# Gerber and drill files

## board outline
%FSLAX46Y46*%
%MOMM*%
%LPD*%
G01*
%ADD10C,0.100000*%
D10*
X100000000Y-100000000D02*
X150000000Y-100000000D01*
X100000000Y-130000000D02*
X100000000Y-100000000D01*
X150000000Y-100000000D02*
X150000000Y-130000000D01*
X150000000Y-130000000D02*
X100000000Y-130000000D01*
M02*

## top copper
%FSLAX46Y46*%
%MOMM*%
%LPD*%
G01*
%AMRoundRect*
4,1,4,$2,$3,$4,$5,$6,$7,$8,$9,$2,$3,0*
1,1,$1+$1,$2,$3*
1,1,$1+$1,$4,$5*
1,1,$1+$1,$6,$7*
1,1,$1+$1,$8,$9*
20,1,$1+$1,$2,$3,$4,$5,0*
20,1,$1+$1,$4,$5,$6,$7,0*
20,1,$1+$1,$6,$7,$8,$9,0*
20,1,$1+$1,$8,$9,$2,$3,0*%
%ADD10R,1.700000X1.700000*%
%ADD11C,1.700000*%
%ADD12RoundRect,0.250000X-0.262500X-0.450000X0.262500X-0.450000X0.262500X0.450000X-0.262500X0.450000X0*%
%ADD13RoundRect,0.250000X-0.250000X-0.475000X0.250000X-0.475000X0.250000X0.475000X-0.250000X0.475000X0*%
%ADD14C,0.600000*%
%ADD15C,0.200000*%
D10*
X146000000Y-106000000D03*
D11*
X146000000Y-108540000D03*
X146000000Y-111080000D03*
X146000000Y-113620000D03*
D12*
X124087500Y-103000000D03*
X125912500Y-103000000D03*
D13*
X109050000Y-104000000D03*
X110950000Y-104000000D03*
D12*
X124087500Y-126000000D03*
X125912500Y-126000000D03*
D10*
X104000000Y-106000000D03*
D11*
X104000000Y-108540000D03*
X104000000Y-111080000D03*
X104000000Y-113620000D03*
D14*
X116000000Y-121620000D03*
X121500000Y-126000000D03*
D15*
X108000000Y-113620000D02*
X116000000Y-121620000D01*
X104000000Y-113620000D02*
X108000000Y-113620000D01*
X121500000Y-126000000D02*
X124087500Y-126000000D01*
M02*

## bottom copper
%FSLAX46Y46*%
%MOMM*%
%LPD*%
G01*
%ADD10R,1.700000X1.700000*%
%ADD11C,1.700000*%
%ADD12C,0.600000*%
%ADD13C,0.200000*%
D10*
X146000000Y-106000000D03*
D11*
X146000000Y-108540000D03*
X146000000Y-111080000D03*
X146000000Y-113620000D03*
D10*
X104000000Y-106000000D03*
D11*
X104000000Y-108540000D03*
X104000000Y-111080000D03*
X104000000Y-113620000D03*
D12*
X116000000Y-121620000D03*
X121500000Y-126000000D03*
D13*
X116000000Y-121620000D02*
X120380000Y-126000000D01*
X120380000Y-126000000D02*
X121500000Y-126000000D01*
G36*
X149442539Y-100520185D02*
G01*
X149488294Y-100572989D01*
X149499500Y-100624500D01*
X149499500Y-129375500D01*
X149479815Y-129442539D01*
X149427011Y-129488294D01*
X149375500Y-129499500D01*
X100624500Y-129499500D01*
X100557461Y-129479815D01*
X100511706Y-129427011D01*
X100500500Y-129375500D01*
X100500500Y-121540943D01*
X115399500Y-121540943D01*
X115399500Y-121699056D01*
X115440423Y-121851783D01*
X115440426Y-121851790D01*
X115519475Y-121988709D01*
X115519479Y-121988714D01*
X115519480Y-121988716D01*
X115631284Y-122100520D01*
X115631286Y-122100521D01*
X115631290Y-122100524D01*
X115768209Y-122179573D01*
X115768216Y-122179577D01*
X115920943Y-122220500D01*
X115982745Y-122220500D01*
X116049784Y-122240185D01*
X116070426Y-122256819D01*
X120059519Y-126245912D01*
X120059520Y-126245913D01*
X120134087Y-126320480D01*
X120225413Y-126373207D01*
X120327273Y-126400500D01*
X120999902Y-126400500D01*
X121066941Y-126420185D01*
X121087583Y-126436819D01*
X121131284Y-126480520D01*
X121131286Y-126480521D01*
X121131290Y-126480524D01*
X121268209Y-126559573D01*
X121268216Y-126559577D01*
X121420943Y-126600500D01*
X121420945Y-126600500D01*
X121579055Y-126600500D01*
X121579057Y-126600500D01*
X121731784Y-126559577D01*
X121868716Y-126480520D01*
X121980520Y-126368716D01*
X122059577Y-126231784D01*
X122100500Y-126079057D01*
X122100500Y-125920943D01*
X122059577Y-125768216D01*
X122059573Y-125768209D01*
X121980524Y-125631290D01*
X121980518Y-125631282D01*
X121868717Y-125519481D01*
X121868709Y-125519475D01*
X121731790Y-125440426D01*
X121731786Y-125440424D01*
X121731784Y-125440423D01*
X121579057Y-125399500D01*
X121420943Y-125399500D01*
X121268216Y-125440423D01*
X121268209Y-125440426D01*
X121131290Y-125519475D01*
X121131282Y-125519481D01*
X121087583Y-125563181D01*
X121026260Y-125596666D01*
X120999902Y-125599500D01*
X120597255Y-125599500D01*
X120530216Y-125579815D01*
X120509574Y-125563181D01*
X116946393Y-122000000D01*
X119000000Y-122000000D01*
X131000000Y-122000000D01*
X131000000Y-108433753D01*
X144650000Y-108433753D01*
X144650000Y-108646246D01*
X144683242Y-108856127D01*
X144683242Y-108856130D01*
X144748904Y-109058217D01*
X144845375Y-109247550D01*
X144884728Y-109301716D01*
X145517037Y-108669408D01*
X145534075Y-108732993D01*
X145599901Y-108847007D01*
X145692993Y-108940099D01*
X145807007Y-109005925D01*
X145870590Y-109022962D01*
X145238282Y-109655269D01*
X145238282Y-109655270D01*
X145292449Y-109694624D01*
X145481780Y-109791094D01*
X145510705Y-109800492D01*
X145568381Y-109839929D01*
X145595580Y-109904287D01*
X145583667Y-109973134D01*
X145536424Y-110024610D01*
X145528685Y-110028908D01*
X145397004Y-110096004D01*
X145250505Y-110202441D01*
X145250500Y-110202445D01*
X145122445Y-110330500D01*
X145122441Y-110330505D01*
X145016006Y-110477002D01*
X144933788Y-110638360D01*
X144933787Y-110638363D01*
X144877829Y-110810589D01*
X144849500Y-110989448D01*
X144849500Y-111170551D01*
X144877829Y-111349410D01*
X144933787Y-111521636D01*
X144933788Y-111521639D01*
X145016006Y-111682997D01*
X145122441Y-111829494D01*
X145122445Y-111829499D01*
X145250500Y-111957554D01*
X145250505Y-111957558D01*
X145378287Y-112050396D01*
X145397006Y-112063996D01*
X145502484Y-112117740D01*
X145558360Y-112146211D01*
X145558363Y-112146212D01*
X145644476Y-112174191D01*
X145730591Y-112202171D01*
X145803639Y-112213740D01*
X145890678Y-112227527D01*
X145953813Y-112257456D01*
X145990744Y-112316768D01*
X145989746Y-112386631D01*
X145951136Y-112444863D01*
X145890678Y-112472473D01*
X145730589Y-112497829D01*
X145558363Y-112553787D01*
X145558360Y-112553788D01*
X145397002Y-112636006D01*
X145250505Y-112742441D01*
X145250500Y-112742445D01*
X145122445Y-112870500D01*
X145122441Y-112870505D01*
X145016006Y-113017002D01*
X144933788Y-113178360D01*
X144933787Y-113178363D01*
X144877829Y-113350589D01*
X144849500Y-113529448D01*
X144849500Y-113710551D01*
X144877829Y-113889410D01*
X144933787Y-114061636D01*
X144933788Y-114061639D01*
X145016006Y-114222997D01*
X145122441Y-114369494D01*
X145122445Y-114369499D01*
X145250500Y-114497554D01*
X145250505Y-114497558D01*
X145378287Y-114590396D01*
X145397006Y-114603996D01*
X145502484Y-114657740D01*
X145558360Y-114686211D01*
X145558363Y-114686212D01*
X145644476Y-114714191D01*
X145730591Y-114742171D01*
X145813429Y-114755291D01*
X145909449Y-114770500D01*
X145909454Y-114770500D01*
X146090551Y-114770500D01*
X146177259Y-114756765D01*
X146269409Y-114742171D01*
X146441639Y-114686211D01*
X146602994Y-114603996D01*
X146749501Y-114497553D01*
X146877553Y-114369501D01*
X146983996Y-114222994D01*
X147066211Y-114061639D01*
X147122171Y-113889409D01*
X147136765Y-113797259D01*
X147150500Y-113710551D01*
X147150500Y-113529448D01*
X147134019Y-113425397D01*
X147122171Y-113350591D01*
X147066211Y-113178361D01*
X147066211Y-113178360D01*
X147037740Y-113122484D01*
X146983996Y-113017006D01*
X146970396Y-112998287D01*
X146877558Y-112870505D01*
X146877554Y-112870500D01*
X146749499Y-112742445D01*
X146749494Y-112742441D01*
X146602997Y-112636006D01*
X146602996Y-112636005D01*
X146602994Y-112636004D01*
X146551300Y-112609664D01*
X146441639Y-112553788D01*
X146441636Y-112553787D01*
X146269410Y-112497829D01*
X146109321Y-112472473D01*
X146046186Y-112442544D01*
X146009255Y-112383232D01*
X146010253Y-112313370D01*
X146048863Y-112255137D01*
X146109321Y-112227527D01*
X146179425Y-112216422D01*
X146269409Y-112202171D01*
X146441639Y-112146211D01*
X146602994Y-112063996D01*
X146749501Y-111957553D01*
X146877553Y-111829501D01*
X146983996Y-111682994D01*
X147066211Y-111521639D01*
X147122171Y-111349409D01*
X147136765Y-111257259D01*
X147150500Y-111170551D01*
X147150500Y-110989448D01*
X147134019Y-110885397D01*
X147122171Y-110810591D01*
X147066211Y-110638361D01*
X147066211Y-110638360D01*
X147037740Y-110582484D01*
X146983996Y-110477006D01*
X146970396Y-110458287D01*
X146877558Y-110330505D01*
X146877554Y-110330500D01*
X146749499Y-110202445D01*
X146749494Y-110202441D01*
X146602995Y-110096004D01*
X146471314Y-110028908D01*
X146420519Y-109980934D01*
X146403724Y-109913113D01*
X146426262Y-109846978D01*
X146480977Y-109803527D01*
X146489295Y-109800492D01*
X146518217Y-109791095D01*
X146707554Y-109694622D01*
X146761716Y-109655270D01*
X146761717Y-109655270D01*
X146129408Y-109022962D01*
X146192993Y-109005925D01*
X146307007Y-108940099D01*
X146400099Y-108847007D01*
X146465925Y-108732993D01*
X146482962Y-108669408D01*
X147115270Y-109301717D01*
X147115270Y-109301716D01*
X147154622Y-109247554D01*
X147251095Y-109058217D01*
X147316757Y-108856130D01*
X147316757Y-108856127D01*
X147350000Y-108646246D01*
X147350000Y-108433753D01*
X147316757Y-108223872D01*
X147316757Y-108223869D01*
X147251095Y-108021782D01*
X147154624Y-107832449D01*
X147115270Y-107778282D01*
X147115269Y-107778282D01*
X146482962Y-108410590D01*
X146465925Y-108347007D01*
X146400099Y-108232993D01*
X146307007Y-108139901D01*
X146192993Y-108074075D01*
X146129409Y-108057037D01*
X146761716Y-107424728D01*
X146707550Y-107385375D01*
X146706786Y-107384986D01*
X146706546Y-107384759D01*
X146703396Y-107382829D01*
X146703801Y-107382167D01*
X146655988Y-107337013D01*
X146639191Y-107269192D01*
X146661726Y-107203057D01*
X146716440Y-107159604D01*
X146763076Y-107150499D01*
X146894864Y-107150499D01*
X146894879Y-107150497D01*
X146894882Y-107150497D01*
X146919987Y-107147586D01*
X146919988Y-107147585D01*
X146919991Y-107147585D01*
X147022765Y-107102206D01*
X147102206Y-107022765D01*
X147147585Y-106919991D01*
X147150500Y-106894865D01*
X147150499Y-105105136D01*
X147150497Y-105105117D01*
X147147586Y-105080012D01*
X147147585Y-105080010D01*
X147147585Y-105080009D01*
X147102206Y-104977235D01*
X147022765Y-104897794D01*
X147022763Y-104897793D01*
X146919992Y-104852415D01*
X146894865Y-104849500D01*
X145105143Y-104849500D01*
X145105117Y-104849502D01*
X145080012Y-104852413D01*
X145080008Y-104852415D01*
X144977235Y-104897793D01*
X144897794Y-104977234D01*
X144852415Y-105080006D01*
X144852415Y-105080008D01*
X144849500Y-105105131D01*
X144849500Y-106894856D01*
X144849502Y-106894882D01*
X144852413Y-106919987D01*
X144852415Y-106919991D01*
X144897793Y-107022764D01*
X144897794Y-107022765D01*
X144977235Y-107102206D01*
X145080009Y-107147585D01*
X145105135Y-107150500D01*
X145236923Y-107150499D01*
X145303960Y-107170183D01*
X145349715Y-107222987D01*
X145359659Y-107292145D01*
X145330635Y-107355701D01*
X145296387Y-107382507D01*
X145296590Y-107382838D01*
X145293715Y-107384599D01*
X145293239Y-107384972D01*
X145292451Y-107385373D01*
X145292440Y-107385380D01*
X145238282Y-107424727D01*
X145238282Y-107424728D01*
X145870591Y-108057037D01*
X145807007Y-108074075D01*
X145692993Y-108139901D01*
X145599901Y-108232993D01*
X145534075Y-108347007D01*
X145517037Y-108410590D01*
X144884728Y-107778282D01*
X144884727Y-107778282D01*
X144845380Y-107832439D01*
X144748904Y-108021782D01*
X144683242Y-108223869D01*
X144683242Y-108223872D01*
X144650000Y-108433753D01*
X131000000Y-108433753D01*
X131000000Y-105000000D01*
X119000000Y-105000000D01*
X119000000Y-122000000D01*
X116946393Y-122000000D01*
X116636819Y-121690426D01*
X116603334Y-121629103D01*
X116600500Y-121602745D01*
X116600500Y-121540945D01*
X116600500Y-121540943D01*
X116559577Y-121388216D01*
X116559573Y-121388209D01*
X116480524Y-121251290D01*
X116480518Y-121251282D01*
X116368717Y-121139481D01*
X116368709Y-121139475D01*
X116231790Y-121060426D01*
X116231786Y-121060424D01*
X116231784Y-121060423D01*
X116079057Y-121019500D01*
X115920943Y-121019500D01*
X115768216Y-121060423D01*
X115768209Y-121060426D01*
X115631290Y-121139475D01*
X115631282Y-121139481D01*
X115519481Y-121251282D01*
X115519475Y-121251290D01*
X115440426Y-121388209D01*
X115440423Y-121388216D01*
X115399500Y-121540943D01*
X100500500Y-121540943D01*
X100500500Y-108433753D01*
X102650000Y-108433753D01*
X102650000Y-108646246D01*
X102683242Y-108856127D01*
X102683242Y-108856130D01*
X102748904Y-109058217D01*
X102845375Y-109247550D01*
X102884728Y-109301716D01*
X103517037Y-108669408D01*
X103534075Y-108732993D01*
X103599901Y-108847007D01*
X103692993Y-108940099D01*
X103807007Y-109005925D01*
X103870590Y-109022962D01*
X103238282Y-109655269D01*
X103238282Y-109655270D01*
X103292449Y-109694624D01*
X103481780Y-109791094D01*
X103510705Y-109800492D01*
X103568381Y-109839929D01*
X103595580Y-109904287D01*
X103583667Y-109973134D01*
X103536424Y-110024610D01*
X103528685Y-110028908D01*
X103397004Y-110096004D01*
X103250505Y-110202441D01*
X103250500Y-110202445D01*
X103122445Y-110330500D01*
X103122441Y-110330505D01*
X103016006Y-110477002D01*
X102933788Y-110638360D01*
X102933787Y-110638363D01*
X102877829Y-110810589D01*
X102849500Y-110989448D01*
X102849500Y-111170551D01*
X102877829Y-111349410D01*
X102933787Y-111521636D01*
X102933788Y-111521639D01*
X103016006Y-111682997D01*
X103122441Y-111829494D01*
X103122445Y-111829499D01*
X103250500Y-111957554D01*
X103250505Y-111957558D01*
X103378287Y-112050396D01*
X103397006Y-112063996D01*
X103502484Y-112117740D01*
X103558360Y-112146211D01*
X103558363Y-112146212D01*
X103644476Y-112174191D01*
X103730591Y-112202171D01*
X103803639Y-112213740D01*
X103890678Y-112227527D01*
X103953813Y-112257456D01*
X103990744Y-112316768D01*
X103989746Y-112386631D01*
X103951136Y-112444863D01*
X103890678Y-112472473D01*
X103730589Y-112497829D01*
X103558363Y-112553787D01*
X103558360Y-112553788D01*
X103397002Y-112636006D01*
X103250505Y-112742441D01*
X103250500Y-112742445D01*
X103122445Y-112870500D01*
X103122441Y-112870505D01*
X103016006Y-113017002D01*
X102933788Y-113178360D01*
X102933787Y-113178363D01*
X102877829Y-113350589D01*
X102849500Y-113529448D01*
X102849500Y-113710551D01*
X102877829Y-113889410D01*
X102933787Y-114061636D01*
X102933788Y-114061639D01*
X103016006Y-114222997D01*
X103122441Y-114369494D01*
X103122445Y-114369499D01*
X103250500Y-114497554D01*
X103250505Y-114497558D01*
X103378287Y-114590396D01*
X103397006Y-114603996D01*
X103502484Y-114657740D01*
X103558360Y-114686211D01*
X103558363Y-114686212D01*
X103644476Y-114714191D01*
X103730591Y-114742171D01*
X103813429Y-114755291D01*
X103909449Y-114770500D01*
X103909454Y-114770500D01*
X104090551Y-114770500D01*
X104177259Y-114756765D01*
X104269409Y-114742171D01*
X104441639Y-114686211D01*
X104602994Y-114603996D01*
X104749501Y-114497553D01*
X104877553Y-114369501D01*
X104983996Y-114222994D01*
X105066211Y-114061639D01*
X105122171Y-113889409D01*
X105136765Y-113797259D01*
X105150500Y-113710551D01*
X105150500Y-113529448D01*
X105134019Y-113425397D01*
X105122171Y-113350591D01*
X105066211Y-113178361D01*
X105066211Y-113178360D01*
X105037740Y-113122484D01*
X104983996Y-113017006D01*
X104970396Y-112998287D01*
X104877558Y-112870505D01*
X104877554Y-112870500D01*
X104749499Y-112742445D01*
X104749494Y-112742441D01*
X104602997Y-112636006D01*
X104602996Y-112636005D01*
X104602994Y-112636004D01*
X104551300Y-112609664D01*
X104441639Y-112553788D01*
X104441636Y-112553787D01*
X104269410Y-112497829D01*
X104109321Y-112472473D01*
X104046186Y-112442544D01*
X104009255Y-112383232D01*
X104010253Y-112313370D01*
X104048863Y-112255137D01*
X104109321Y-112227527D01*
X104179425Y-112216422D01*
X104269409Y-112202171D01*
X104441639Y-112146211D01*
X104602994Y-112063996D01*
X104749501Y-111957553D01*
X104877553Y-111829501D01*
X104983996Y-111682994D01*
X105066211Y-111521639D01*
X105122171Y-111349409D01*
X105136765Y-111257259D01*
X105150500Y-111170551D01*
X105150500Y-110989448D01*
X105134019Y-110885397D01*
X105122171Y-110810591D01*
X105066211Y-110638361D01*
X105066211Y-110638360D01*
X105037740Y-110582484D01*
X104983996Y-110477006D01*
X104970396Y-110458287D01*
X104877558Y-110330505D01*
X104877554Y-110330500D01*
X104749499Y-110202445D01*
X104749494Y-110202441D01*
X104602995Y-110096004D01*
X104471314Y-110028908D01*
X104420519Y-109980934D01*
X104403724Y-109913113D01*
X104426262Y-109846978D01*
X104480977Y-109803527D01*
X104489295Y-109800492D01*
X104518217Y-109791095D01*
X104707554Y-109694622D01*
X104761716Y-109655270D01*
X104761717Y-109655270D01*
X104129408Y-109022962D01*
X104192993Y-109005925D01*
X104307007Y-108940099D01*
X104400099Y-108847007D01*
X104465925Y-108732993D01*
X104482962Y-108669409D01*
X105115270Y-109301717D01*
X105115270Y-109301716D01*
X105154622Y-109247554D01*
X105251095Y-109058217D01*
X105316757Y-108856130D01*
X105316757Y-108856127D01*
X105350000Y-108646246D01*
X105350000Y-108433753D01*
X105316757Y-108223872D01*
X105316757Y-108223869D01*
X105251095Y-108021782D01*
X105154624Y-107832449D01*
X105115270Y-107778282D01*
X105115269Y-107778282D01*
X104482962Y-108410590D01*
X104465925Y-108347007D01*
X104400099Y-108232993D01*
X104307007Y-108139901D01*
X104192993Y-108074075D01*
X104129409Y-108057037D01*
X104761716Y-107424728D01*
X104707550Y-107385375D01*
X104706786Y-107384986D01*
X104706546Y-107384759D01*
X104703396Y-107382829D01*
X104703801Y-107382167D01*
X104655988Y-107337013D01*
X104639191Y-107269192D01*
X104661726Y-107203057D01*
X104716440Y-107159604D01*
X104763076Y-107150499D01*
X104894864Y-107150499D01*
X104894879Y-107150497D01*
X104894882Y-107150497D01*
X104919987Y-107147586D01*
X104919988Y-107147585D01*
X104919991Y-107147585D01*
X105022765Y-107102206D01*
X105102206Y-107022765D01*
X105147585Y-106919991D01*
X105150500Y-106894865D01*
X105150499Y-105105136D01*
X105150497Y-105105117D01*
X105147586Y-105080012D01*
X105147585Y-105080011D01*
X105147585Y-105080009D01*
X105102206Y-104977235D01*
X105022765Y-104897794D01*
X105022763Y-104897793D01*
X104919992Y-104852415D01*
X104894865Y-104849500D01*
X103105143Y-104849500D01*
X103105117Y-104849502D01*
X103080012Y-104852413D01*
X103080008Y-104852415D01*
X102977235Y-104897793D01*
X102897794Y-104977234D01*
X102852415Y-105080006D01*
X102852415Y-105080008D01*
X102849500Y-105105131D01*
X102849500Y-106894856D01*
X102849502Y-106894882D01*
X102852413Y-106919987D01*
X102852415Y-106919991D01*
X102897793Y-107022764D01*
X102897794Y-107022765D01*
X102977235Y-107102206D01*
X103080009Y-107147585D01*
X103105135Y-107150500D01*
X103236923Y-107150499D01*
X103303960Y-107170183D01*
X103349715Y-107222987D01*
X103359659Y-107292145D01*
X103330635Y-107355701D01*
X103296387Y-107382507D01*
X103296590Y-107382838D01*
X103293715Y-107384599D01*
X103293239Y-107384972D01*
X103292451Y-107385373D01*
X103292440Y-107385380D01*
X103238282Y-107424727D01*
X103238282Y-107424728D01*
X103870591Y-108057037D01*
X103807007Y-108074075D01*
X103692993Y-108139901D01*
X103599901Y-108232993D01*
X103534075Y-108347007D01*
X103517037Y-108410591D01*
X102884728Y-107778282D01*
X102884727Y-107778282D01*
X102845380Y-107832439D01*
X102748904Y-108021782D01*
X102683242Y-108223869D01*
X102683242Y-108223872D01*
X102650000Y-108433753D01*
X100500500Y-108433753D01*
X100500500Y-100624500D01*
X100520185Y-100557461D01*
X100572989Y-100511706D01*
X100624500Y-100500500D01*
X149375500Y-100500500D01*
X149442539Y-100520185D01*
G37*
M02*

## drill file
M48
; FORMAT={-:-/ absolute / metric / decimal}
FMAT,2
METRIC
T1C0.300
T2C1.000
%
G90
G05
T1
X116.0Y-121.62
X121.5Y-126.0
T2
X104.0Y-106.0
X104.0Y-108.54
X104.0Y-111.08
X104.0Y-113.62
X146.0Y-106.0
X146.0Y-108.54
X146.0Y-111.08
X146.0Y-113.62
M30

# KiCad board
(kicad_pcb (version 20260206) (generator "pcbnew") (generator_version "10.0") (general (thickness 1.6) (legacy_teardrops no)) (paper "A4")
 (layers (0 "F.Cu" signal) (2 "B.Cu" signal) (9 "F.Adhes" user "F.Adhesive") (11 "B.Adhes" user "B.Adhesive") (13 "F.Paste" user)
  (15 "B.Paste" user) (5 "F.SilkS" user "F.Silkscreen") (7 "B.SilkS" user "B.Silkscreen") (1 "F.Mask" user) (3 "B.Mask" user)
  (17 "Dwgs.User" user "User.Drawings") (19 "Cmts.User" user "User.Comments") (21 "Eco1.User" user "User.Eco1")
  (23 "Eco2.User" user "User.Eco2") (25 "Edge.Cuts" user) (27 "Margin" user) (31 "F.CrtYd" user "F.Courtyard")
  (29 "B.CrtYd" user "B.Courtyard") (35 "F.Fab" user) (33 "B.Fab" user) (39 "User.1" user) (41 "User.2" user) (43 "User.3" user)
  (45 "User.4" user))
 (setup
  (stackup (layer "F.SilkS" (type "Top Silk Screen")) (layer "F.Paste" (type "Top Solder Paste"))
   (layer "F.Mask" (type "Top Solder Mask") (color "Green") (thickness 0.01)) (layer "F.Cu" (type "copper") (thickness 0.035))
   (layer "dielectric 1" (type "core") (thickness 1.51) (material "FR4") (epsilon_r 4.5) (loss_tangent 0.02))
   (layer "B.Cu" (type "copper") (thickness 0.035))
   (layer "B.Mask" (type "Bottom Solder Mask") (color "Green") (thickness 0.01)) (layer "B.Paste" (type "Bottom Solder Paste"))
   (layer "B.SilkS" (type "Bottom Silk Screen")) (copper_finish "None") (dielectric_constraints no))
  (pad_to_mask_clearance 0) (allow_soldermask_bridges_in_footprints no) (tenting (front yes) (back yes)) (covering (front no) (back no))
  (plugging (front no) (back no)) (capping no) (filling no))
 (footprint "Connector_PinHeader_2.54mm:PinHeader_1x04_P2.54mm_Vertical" (layer "F.Cu") (at 146 106)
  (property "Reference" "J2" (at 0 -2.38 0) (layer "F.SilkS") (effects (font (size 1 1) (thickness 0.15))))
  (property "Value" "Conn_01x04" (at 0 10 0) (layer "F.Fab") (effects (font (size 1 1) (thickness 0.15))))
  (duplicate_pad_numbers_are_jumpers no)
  (pad "1" thru_hole rect (at 0 0) (size 1.7 1.7) (drill 1) (layers "*.Cu" "*.Mask") (remove_unused_layers no) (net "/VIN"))
  (pad "2" thru_hole circle (at 0 2.54) (size 1.7 1.7) (drill 1) (layers "*.Cu" "*.Mask") (remove_unused_layers no) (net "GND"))
  (pad "3" thru_hole circle (at 0 5.08) (size 1.7 1.7) (drill 1) (layers "*.Cu" "*.Mask") (remove_unused_layers no) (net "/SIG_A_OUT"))
  (pad "4" thru_hole circle (at 0 7.62) (size 1.7 1.7) (drill 1) (layers "*.Cu" "*.Mask") (remove_unused_layers no) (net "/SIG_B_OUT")))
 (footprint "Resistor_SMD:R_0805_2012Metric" (layer "F.Cu") (at 125 103)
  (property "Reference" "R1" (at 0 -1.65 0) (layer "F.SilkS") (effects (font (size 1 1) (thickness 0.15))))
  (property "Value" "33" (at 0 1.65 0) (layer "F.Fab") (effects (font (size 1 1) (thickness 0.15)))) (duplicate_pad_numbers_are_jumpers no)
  (pad "1" smd roundrect (at -0.9125 0) (size 1.025 1.4) (layers "F.Cu" "F.Mask" "F.Paste") (roundrect_rratio 0.243902) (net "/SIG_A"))
  (pad "2" smd roundrect (at 0.9125 0) (size 1.025 1.4) (layers "F.Cu" "F.Mask" "F.Paste") (roundrect_rratio 0.243902) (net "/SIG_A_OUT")))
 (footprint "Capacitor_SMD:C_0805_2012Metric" (layer "F.Cu") (at 110 104)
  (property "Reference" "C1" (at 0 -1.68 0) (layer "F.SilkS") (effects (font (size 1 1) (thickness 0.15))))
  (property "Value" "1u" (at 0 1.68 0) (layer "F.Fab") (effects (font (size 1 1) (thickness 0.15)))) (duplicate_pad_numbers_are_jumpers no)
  (pad "1" smd roundrect (at -0.95 0) (size 1 1.45) (layers "F.Cu" "F.Mask" "F.Paste") (roundrect_rratio 0.25) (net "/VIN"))
  (pad "2" smd roundrect (at 0.95 0) (size 1 1.45) (layers "F.Cu" "F.Mask" "F.Paste") (roundrect_rratio 0.25) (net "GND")))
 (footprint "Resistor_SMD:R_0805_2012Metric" (layer "F.Cu") (at 125 126)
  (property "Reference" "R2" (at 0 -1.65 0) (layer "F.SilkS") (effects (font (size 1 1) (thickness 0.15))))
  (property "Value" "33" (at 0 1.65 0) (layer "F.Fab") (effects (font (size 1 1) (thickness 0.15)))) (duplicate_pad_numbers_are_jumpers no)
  (pad "1" smd roundrect (at -0.9125 0) (size 1.025 1.4) (layers "F.Cu" "F.Mask" "F.Paste") (roundrect_rratio 0.243902) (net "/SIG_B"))
  (pad "2" smd roundrect (at 0.9125 0) (size 1.025 1.4) (layers "F.Cu" "F.Mask" "F.Paste") (roundrect_rratio 0.243902) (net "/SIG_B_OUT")))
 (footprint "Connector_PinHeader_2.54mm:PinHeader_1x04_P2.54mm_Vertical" (layer "F.Cu") (at 104 106)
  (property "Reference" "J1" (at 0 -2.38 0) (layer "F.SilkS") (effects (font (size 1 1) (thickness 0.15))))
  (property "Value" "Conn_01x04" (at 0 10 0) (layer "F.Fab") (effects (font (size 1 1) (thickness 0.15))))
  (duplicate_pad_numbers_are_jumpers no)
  (pad "1" thru_hole rect (at 0 0) (size 1.7 1.7) (drill 1) (layers "*.Cu" "*.Mask") (remove_unused_layers no) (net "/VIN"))
  (pad "2" thru_hole circle (at 0 2.54) (size 1.7 1.7) (drill 1) (layers "*.Cu" "*.Mask") (remove_unused_layers no) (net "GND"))
  (pad "3" thru_hole circle (at 0 5.08) (size 1.7 1.7) (drill 1) (layers "*.Cu" "*.Mask") (remove_unused_layers no) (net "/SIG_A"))
  (pad "4" thru_hole circle (at 0 7.62) (size 1.7 1.7) (drill 1) (layers "*.Cu" "*.Mask") (remove_unused_layers no) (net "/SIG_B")))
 (gr_line (start 100 100) (end 150 100) (stroke (width 0.1) (type default)) (layer "Edge.Cuts"))
 (gr_line (start 100 130) (end 100 100) (stroke (width 0.1) (type default)) (layer "Edge.Cuts"))
 (gr_line (start 150 100) (end 150 130) (stroke (width 0.1) (type default)) (layer "Edge.Cuts"))
 (gr_line (start 150 130) (end 100 130) (stroke (width 0.1) (type default)) (layer "Edge.Cuts"))
 (segment (start 108 113.62) (end 116 121.62) (width 0.2) (locked yes) (layer "F.Cu") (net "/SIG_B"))
 (segment (start 104 113.62) (end 108 113.62) (width 0.2) (locked yes) (layer "F.Cu") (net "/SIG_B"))
 (segment (start 121.5 126) (end 124.0875 126) (width 0.2) (locked yes) (layer "F.Cu") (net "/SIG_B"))
 (via (at 116 121.62) (size 0.6) (drill 0.3) (layers "F.Cu" "B.Cu") (locked yes) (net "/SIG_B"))
 (via (at 121.5 126) (size 0.6) (drill 0.3) (layers "F.Cu" "B.Cu") (locked yes) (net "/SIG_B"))
 (segment (start 116 121.62) (end 120.38 126) (width 0.2) (locked yes) (layer "B.Cu") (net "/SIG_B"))
 (segment (start 120.38 126) (end 121.5 126) (width 0.2) (locked yes) (layer "B.Cu") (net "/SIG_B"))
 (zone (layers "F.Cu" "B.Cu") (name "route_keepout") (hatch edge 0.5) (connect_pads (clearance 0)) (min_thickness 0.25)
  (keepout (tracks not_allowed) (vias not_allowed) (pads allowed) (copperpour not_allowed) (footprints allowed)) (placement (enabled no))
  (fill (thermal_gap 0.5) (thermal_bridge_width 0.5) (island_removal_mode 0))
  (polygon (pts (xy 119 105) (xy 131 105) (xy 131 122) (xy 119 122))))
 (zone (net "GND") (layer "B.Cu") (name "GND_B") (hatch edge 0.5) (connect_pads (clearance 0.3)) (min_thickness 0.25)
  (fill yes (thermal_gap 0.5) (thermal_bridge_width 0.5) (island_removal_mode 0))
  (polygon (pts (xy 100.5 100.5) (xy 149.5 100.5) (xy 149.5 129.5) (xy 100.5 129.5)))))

